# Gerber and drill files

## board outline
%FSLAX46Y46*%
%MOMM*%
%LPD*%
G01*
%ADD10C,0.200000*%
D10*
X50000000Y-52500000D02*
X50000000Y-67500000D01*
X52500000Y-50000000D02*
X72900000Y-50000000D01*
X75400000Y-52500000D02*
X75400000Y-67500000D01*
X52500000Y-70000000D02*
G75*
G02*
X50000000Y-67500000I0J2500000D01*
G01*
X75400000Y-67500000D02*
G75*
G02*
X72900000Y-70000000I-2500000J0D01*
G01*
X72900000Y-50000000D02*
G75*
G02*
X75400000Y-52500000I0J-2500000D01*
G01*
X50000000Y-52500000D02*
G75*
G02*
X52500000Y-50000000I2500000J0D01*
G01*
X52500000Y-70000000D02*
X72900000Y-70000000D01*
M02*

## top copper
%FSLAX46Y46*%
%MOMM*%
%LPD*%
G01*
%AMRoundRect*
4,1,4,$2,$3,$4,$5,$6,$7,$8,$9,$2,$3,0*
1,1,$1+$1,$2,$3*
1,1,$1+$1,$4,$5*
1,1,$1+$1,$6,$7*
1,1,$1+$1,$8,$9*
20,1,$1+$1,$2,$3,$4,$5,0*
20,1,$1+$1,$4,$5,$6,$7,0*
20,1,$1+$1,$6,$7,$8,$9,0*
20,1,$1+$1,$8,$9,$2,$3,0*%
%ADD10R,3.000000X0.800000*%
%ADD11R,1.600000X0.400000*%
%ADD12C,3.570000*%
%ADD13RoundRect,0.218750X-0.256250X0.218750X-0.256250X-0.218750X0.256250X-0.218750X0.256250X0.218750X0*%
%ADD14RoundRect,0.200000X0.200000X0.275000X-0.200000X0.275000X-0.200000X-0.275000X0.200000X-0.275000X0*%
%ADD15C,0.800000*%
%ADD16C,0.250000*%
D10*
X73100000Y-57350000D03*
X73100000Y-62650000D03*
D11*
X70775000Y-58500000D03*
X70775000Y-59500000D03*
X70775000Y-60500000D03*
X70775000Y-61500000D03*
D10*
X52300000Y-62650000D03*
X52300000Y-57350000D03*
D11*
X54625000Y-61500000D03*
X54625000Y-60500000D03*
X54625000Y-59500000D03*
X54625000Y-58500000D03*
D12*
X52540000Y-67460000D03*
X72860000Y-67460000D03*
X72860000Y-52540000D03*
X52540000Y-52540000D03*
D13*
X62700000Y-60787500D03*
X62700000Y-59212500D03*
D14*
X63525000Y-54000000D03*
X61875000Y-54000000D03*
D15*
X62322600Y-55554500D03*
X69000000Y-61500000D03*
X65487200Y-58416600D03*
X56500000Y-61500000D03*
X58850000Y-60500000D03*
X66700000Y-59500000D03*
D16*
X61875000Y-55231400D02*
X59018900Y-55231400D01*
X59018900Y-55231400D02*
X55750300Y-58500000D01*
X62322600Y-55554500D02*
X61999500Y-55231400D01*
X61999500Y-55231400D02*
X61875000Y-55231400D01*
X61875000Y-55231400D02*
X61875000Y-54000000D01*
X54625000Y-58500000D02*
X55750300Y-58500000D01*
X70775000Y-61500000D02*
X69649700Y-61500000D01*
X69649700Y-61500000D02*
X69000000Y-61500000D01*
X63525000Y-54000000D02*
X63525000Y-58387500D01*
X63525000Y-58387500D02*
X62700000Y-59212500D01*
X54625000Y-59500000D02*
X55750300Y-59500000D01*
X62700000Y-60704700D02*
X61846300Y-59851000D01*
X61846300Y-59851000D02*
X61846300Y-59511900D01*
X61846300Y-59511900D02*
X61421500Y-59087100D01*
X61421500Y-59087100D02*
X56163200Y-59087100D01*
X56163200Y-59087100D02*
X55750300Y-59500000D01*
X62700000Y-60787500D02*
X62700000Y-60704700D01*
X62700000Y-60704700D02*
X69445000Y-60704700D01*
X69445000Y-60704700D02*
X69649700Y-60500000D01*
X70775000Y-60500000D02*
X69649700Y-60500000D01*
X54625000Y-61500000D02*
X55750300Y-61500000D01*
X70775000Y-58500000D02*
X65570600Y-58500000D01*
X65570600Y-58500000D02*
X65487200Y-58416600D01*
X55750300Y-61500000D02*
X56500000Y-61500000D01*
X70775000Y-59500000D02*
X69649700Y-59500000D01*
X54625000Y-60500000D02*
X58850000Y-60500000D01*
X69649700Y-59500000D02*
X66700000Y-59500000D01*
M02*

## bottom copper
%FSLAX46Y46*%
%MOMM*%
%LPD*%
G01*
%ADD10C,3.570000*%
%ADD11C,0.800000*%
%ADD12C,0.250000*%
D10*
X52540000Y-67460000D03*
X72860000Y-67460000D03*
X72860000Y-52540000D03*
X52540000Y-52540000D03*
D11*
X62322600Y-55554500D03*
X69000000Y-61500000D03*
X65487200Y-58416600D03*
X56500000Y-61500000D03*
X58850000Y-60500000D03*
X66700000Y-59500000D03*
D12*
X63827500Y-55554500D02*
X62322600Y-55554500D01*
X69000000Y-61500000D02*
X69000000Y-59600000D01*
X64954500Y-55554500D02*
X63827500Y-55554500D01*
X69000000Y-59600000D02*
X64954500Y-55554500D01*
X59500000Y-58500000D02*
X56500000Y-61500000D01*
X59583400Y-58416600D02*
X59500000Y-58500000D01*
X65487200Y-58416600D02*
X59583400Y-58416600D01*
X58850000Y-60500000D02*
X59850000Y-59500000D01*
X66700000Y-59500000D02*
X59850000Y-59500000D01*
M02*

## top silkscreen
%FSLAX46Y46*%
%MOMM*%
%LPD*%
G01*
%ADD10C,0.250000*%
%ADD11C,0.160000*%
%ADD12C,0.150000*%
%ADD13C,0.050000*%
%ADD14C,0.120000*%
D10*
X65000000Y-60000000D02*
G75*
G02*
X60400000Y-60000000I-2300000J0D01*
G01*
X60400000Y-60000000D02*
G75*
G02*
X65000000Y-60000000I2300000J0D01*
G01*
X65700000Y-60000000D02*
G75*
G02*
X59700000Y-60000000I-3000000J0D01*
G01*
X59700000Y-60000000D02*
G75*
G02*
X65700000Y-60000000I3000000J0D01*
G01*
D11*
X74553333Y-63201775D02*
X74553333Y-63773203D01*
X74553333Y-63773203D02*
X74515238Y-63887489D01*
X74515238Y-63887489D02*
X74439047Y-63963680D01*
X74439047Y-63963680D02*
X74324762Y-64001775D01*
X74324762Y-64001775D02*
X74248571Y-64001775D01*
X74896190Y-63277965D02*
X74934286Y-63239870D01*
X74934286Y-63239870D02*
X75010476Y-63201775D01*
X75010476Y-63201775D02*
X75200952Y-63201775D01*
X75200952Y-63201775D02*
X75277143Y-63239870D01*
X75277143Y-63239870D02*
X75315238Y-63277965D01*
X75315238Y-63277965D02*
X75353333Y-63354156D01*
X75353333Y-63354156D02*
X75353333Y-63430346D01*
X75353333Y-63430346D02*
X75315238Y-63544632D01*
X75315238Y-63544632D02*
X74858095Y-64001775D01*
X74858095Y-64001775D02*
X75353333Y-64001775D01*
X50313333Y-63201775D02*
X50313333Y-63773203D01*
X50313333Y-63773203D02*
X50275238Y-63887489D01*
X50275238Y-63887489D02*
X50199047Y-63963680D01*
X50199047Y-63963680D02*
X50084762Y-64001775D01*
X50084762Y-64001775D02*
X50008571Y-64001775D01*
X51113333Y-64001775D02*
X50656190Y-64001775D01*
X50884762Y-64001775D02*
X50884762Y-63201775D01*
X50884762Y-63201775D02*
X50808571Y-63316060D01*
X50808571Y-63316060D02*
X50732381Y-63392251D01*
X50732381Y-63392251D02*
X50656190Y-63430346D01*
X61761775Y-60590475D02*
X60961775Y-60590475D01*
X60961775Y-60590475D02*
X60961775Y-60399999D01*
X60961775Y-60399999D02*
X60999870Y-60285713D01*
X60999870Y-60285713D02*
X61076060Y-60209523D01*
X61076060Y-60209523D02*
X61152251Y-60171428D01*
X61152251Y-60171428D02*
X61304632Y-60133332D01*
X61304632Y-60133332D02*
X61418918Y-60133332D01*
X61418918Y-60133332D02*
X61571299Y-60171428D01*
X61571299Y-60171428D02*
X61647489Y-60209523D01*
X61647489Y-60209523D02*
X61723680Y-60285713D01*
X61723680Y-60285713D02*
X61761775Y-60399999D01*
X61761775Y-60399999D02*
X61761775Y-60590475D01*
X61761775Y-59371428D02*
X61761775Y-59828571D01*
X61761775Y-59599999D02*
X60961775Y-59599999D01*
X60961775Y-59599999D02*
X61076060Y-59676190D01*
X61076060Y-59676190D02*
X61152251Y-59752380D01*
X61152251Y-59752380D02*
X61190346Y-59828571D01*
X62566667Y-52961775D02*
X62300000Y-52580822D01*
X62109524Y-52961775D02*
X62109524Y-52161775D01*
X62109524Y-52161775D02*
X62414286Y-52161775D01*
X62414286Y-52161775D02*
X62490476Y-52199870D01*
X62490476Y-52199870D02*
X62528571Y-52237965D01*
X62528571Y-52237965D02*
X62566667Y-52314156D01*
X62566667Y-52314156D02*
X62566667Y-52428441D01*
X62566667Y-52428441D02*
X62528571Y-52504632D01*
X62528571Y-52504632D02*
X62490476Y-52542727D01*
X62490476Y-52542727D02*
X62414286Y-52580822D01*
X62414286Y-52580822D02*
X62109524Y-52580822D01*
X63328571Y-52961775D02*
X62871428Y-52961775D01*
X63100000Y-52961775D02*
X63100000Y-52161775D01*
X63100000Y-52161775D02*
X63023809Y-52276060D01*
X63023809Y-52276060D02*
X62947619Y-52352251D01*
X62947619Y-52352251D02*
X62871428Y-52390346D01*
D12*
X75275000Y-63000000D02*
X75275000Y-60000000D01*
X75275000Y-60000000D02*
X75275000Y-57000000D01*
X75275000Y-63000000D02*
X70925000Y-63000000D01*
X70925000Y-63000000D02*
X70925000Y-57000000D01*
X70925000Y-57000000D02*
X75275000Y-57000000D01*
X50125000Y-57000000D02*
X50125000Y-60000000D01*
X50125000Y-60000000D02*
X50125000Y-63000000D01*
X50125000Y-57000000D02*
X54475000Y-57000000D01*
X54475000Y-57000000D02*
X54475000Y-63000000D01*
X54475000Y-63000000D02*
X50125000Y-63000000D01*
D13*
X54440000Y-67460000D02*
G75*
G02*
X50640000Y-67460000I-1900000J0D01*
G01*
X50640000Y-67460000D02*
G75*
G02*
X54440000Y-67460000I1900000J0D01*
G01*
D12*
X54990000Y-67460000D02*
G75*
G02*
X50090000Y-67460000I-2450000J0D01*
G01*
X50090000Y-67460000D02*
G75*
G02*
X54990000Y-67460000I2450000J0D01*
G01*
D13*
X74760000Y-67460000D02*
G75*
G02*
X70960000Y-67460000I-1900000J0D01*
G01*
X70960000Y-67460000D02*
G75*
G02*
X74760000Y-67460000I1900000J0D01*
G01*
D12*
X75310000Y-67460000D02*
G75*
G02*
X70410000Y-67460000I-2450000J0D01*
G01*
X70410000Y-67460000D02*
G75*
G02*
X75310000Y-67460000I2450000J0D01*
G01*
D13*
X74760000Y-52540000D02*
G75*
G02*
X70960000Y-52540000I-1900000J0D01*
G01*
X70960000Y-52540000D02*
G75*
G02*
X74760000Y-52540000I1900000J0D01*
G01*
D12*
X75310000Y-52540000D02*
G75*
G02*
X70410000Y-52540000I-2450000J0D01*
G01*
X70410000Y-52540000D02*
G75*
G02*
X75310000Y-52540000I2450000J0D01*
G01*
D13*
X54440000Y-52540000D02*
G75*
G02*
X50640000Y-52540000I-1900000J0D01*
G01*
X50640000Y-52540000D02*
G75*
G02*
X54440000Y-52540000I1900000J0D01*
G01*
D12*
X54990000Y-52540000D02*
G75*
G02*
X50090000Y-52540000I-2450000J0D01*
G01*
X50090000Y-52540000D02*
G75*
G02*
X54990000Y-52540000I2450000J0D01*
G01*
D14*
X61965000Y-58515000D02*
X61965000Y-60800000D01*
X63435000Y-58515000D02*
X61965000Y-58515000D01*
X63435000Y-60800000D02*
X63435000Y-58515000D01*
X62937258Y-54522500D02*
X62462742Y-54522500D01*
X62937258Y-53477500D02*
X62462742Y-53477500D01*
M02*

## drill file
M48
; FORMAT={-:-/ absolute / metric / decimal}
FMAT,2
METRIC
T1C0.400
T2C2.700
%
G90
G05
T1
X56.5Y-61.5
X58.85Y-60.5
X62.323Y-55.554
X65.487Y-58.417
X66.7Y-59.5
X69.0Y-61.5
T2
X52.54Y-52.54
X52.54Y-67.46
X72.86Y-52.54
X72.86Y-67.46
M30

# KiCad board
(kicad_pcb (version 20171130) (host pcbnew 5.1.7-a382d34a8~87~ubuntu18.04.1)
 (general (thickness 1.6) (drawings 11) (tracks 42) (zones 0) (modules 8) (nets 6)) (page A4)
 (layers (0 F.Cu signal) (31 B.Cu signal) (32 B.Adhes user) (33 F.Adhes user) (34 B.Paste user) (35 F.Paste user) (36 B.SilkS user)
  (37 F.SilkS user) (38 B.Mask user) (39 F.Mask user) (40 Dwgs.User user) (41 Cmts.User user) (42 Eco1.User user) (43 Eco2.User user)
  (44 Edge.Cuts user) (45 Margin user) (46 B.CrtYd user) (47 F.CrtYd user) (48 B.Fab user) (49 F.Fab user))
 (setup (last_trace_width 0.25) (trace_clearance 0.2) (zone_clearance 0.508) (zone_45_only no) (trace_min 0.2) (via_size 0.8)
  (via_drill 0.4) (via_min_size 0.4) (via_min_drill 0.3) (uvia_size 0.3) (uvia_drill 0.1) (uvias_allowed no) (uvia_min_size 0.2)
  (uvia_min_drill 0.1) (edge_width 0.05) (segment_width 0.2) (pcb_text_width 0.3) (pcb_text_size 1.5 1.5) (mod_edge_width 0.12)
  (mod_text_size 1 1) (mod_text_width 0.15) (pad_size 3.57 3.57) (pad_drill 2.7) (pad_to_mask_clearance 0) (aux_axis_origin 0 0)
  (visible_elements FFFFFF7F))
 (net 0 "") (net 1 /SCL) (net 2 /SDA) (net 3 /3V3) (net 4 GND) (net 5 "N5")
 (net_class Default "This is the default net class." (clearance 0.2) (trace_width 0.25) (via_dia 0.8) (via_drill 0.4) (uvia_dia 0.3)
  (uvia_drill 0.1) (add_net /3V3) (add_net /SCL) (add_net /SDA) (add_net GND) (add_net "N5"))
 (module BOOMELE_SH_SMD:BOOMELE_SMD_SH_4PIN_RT (layer F.Cu) (at 72.62 60 270)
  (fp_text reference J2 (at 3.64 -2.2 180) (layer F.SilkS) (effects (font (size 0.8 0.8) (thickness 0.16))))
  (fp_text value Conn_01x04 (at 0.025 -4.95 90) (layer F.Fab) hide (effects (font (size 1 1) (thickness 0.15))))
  (fp_line (start 3 -2.655) (end 0 -2.655) (layer F.SilkS) (width 0.15))
  (fp_line (start 0 -2.655) (end -3 -2.655) (layer F.SilkS) (width 0.15))
  (fp_line (start 3 -2.655) (end 3 1.695) (layer F.SilkS) (width 0.15))
  (fp_line (start 3 1.695) (end -3 1.695) (layer F.SilkS) (width 0.15))
  (fp_line (start -3 1.695) (end -3 -2.655) (layer F.SilkS) (width 0.15))
  (pad "" smd rect (at -2.65 -0.48 90) (size 0.8 3) (layers F.Cu F.Paste F.Mask))
  (pad "" smd rect (at 2.65 -0.48 90) (size 0.8 3) (layers F.Cu F.Paste F.Mask))
  (pad 4 smd rect (at -1.5 1.845 90) (size 0.4 1.6) (layers F.Cu F.Paste F.Mask) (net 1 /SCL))
  (pad 3 smd rect (at -0.5 1.845 90) (size 0.4 1.6) (layers F.Cu F.Paste F.Mask) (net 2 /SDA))
  (pad 2 smd rect (at 0.5 1.845 90) (size 0.4 1.6) (layers F.Cu F.Paste F.Mask) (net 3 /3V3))
  (pad 1 smd rect (at 1.5 1.845 90) (size 0.4 1.6) (layers F.Cu F.Paste F.Mask) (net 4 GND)))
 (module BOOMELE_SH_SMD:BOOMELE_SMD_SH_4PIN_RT (layer F.Cu) (at 52.78 60 90)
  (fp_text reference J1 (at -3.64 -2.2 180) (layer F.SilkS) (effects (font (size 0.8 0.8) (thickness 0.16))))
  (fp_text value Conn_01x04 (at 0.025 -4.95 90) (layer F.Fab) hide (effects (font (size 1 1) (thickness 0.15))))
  (fp_line (start 3 -2.655) (end 0 -2.655) (layer F.SilkS) (width 0.15))
  (fp_line (start 0 -2.655) (end -3 -2.655) (layer F.SilkS) (width 0.15))
  (fp_line (start 3 -2.655) (end 3 1.695) (layer F.SilkS) (width 0.15))
  (fp_line (start 3 1.695) (end -3 1.695) (layer F.SilkS) (width 0.15))
  (fp_line (start -3 1.695) (end -3 -2.655) (layer F.SilkS) (width 0.15))
  (pad "" smd rect (at -2.65 -0.48 270) (size 0.8 3) (layers F.Cu F.Paste F.Mask))
  (pad "" smd rect (at 2.65 -0.48 270) (size 0.8 3) (layers F.Cu F.Paste F.Mask))
  (pad 4 smd rect (at -1.5 1.845 270) (size 0.4 1.6) (layers F.Cu F.Paste F.Mask) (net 1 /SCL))
  (pad 3 smd rect (at -0.5 1.845 270) (size 0.4 1.6) (layers F.Cu F.Paste F.Mask) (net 2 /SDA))
  (pad 2 smd rect (at 0.5 1.845 270) (size 0.4 1.6) (layers F.Cu F.Paste F.Mask) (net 3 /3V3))
  (pad 1 smd rect (at 1.5 1.845 270) (size 0.4 1.6) (layers F.Cu F.Paste F.Mask) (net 4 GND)))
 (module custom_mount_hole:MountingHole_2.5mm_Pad (layer F.Cu) (at 52.54 67.46)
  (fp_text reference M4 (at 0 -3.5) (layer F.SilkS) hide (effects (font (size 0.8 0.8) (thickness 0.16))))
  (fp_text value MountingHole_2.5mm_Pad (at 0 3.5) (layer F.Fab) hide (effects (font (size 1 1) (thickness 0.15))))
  (fp_circle (center 0 0) (end 1.9 0) (layer F.SilkS) (width 0.05))
  (fp_circle (center 0 0) (end 2.45 0) (layer F.SilkS) (width 0.15))
  (pad ~ thru_hole circle (at 0 0) (size 3.57 3.57) (drill 2.7) (layers *.Cu *.Mask)))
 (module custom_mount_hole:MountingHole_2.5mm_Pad (layer F.Cu) (at 72.86 67.46)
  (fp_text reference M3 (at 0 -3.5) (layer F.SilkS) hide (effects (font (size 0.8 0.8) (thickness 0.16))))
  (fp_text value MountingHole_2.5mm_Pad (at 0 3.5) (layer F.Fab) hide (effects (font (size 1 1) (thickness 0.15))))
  (fp_circle (center 0 0) (end 1.9 0) (layer F.SilkS) (width 0.05))
  (fp_circle (center 0 0) (end 2.45 0) (layer F.SilkS) (width 0.15))
  (pad ~ thru_hole circle (at 0 0) (size 3.57 3.57) (drill 2.7) (layers *.Cu *.Mask)))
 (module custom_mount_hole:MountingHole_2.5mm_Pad (layer F.Cu) (at 72.86 52.54)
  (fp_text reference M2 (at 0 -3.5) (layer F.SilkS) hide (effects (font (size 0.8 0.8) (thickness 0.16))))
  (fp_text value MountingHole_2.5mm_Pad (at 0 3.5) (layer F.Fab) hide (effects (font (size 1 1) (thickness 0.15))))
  (fp_circle (center 0 0) (end 1.9 0) (layer F.SilkS) (width 0.05))
  (fp_circle (center 0 0) (end 2.45 0) (layer F.SilkS) (width 0.15))
  (pad ~ thru_hole circle (at 0 0) (size 3.57 3.57) (drill 2.7) (layers *.Cu *.Mask)))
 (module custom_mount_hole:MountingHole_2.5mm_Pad (layer F.Cu) (at 52.54 52.54)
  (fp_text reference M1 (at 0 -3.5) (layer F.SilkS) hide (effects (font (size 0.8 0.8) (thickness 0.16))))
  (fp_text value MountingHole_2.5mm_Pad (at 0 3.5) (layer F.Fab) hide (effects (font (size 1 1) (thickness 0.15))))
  (fp_circle (center 0 0) (end 1.9 0) (layer F.SilkS) (width 0.05))
  (fp_circle (center 0 0) (end 2.45 0) (layer F.SilkS) (width 0.15))
  (pad ~ thru_hole circle (at 0 0) (size 3.57 3.57) (drill 2.7) (layers *.Cu *.Mask)))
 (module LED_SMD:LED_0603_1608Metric (layer F.Cu) (at 62.7 60 270)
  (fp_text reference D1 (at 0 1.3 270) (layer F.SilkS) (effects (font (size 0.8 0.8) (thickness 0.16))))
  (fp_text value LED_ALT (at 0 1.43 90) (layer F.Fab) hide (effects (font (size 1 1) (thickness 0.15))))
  (fp_line (start -1.485 0.735) (end 0.8 0.735) (layer F.SilkS) (width 0.12))
  (fp_line (start -1.485 -0.735) (end -1.485 0.735) (layer F.SilkS) (width 0.12))
  (fp_line (start 0.8 -0.735) (end -1.485 -0.735) (layer F.SilkS) (width 0.12))
  (pad 2 smd roundrect (at 0.7875 0 270) (size 0.875 0.95) (layers F.Cu F.Paste F.Mask) (roundrect_rratio 0.25) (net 3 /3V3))
  (pad 1 smd roundrect (at -0.7875 0 270) (size 0.875 0.95) (layers F.Cu F.Paste F.Mask) (roundrect_rratio 0.25) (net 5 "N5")))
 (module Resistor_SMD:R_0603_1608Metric (layer F.Cu) (at 62.7 54 180)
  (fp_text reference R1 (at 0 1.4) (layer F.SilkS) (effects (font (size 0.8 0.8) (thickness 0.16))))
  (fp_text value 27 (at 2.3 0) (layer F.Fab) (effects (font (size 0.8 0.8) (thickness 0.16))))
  (fp_line (start -0.237258 -0.5225) (end 0.237258 -0.5225) (layer F.SilkS) (width 0.12))
  (fp_line (start -0.237258 0.5225) (end 0.237258 0.5225) (layer F.SilkS) (width 0.12))
  (pad 1 smd roundrect (at -0.825 0 180) (size 0.8 0.95) (layers F.Cu F.Paste F.Mask) (roundrect_rratio 0.25) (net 5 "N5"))
  (pad 2 smd roundrect (at 0.825 0 180) (size 0.8 0.95) (layers F.Cu F.Paste F.Mask) (roundrect_rratio 0.25) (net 4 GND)))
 (gr_circle (center 62.7 60) (end 65 60) (layer F.SilkS) (width 0.25))
 (gr_circle (center 62.7 60) (end 65.7 60) (layer F.SilkS) (width 0.25))
 (gr_line (start 50 52.5) (end 50 67.5) (layer Edge.Cuts) (width 0.2))
 (gr_line (start 52.5 50) (end 72.9 50) (layer Edge.Cuts) (width 0.2))
 (gr_line (start 75.4 52.5) (end 75.4 67.5) (layer Edge.Cuts) (width 0.2))
 (gr_arc (start 52.5 67.5) (end 50 67.5) (angle -90) (layer Edge.Cuts) (width 0.2))
 (gr_arc (start 72.9 67.5) (end 72.9 70) (angle -90) (layer Edge.Cuts) (width 0.2))
 (gr_arc (start 72.9 52.5) (end 75.4 52.5) (angle -90) (layer Edge.Cuts) (width 0.2))
 (gr_arc (start 52.5 52.5) (end 52.5 50) (angle -90) (layer Edge.Cuts) (width 0.2))
 (gr_line (start 52.5 70) (end 72.9 70) (layer Edge.Cuts) (width 0.2))
 (segment (start 63.8275 55.5545) (end 62.3226 55.5545) (width 0.25) (layer B.Cu) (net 4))
 (segment (start 61.875 55.2314) (end 59.0189 55.2314) (width 0.25) (layer F.Cu) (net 4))
 (segment (start 59.0189 55.2314) (end 55.7503 58.5) (width 0.25) (layer F.Cu) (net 4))
 (segment (start 62.3226 55.5545) (end 61.9995 55.2314) (width 0.25) (layer F.Cu) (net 4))
 (segment (start 61.9995 55.2314) (end 61.875 55.2314) (width 0.25) (layer F.Cu) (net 4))
 (segment (start 61.875 55.2314) (end 61.875 54) (width 0.25) (layer F.Cu) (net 4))
 (segment (start 54.625 58.5) (end 55.7503 58.5) (width 0.25) (layer F.Cu) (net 4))
 (segment (start 70.775 61.5) (end 69.6497 61.5) (width 0.25) (layer F.Cu) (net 4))
 (via (at 62.3226 55.5545) (size 0.8) (layers F.Cu B.Cu) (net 4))
 (via (at 69 61.5) (size 0.8) (drill 0.4) (layers F.Cu B.Cu) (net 4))
 (segment (start 69.6497 61.5) (end 69 61.5) (width 0.25) (layer F.Cu) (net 4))
 (segment (start 69 61.5) (end 69 59.6) (width 0.25) (layer B.Cu) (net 4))
 (segment (start 64.9545 55.5545) (end 63.8275 55.5545) (width 0.25) (layer B.Cu) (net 4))
 (segment (start 69 59.6) (end 64.9545 55.5545) (width 0.25) (layer B.Cu) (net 4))
 (segment (start 63.525 54) (end 63.525 58.3875) (width 0.25) (layer F.Cu) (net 5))
 (segment (start 63.525 58.3875) (end 62.7 59.2125) (width 0.25) (layer F.Cu) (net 5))
 (segment (start 54.625 59.5) (end 55.7503 59.5) (width 0.25) (layer F.Cu) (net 3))
 (segment (start 62.7 60.7047) (end 61.8463 59.851) (width 0.25) (layer F.Cu) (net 3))
 (segment (start 61.8463 59.851) (end 61.8463 59.5119) (width 0.25) (layer F.Cu) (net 3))
 (segment (start 61.8463 59.5119) (end 61.4215 59.0871) (width 0.25) (layer F.Cu) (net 3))
 (segment (start 61.4215 59.0871) (end 56.1632 59.0871) (width 0.25) (layer F.Cu) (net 3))
 (segment (start 56.1632 59.0871) (end 55.7503 59.5) (width 0.25) (layer F.Cu) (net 3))
 (segment (start 62.7 60.7875) (end 62.7 60.7047) (width 0.25) (layer F.Cu) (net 3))
 (segment (start 62.7 60.7047) (end 69.445 60.7047) (width 0.25) (layer F.Cu) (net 3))
 (segment (start 69.445 60.7047) (end 69.6497 60.5) (width 0.25) (layer F.Cu) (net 3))
 (segment (start 70.775 60.5) (end 69.6497 60.5) (width 0.25) (layer F.Cu) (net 3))
 (segment (start 54.625 61.5) (end 55.7503 61.5) (width 0.25) (layer F.Cu) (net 1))
 (segment (start 70.775 58.5) (end 65.5706 58.5) (width 0.25) (layer F.Cu) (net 1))
 (segment (start 65.5706 58.5) (end 65.4872 58.4166) (width 0.25) (layer F.Cu) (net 1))
 (via (at 65.4872 58.4166) (size 0.8) (layers F.Cu B.Cu) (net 1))
 (via (at 56.5 61.5) (size 0.8) (drill 0.4) (layers F.Cu B.Cu) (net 1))
 (segment (start 55.7503 61.5) (end 56.5 61.5) (width 0.25) (layer F.Cu) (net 1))
 (segment (start 59.5 58.5) (end 56.5 61.5) (width 0.25) (layer B.Cu) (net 1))
 (segment (start 59.5834 58.4166) (end 59.5 58.5) (width 0.25) (layer B.Cu) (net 1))
 (segment (start 65.4872 58.4166) (end 59.5834 58.4166) (width 0.25) (layer B.Cu) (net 1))
 (segment (start 70.775 59.5) (end 69.6497 59.5) (width 0.25) (layer F.Cu) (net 2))
 (via (at 58.85 60.5) (size 0.8) (drill 0.4) (layers F.Cu B.Cu) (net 2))
 (segment (start 54.625 60.5) (end 58.85 60.5) (width 0.25) (layer F.Cu) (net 2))
 (segment (start 58.85 60.5) (end 59.85 59.5) (width 0.25) (layer B.Cu) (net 2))
 (via (at 66.7 59.5) (size 0.8) (drill 0.4) (layers F.Cu B.Cu) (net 2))
 (segment (start 69.6497 59.5) (end 66.7 59.5) (width 0.25) (layer F.Cu) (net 2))
 (segment (start 66.7 59.5) (end 59.85 59.5) (width 0.25) (layer B.Cu) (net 2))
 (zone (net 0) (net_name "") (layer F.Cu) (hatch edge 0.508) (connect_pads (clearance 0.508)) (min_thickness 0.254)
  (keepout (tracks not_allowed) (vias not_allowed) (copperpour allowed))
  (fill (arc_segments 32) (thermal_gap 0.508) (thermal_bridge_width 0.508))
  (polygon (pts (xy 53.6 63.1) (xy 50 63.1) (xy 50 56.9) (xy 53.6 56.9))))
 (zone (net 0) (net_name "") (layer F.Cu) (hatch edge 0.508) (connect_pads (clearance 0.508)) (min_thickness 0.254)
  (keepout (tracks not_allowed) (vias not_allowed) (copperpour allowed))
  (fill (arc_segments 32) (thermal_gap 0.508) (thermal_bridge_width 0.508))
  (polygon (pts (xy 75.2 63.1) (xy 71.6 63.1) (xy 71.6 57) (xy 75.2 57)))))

